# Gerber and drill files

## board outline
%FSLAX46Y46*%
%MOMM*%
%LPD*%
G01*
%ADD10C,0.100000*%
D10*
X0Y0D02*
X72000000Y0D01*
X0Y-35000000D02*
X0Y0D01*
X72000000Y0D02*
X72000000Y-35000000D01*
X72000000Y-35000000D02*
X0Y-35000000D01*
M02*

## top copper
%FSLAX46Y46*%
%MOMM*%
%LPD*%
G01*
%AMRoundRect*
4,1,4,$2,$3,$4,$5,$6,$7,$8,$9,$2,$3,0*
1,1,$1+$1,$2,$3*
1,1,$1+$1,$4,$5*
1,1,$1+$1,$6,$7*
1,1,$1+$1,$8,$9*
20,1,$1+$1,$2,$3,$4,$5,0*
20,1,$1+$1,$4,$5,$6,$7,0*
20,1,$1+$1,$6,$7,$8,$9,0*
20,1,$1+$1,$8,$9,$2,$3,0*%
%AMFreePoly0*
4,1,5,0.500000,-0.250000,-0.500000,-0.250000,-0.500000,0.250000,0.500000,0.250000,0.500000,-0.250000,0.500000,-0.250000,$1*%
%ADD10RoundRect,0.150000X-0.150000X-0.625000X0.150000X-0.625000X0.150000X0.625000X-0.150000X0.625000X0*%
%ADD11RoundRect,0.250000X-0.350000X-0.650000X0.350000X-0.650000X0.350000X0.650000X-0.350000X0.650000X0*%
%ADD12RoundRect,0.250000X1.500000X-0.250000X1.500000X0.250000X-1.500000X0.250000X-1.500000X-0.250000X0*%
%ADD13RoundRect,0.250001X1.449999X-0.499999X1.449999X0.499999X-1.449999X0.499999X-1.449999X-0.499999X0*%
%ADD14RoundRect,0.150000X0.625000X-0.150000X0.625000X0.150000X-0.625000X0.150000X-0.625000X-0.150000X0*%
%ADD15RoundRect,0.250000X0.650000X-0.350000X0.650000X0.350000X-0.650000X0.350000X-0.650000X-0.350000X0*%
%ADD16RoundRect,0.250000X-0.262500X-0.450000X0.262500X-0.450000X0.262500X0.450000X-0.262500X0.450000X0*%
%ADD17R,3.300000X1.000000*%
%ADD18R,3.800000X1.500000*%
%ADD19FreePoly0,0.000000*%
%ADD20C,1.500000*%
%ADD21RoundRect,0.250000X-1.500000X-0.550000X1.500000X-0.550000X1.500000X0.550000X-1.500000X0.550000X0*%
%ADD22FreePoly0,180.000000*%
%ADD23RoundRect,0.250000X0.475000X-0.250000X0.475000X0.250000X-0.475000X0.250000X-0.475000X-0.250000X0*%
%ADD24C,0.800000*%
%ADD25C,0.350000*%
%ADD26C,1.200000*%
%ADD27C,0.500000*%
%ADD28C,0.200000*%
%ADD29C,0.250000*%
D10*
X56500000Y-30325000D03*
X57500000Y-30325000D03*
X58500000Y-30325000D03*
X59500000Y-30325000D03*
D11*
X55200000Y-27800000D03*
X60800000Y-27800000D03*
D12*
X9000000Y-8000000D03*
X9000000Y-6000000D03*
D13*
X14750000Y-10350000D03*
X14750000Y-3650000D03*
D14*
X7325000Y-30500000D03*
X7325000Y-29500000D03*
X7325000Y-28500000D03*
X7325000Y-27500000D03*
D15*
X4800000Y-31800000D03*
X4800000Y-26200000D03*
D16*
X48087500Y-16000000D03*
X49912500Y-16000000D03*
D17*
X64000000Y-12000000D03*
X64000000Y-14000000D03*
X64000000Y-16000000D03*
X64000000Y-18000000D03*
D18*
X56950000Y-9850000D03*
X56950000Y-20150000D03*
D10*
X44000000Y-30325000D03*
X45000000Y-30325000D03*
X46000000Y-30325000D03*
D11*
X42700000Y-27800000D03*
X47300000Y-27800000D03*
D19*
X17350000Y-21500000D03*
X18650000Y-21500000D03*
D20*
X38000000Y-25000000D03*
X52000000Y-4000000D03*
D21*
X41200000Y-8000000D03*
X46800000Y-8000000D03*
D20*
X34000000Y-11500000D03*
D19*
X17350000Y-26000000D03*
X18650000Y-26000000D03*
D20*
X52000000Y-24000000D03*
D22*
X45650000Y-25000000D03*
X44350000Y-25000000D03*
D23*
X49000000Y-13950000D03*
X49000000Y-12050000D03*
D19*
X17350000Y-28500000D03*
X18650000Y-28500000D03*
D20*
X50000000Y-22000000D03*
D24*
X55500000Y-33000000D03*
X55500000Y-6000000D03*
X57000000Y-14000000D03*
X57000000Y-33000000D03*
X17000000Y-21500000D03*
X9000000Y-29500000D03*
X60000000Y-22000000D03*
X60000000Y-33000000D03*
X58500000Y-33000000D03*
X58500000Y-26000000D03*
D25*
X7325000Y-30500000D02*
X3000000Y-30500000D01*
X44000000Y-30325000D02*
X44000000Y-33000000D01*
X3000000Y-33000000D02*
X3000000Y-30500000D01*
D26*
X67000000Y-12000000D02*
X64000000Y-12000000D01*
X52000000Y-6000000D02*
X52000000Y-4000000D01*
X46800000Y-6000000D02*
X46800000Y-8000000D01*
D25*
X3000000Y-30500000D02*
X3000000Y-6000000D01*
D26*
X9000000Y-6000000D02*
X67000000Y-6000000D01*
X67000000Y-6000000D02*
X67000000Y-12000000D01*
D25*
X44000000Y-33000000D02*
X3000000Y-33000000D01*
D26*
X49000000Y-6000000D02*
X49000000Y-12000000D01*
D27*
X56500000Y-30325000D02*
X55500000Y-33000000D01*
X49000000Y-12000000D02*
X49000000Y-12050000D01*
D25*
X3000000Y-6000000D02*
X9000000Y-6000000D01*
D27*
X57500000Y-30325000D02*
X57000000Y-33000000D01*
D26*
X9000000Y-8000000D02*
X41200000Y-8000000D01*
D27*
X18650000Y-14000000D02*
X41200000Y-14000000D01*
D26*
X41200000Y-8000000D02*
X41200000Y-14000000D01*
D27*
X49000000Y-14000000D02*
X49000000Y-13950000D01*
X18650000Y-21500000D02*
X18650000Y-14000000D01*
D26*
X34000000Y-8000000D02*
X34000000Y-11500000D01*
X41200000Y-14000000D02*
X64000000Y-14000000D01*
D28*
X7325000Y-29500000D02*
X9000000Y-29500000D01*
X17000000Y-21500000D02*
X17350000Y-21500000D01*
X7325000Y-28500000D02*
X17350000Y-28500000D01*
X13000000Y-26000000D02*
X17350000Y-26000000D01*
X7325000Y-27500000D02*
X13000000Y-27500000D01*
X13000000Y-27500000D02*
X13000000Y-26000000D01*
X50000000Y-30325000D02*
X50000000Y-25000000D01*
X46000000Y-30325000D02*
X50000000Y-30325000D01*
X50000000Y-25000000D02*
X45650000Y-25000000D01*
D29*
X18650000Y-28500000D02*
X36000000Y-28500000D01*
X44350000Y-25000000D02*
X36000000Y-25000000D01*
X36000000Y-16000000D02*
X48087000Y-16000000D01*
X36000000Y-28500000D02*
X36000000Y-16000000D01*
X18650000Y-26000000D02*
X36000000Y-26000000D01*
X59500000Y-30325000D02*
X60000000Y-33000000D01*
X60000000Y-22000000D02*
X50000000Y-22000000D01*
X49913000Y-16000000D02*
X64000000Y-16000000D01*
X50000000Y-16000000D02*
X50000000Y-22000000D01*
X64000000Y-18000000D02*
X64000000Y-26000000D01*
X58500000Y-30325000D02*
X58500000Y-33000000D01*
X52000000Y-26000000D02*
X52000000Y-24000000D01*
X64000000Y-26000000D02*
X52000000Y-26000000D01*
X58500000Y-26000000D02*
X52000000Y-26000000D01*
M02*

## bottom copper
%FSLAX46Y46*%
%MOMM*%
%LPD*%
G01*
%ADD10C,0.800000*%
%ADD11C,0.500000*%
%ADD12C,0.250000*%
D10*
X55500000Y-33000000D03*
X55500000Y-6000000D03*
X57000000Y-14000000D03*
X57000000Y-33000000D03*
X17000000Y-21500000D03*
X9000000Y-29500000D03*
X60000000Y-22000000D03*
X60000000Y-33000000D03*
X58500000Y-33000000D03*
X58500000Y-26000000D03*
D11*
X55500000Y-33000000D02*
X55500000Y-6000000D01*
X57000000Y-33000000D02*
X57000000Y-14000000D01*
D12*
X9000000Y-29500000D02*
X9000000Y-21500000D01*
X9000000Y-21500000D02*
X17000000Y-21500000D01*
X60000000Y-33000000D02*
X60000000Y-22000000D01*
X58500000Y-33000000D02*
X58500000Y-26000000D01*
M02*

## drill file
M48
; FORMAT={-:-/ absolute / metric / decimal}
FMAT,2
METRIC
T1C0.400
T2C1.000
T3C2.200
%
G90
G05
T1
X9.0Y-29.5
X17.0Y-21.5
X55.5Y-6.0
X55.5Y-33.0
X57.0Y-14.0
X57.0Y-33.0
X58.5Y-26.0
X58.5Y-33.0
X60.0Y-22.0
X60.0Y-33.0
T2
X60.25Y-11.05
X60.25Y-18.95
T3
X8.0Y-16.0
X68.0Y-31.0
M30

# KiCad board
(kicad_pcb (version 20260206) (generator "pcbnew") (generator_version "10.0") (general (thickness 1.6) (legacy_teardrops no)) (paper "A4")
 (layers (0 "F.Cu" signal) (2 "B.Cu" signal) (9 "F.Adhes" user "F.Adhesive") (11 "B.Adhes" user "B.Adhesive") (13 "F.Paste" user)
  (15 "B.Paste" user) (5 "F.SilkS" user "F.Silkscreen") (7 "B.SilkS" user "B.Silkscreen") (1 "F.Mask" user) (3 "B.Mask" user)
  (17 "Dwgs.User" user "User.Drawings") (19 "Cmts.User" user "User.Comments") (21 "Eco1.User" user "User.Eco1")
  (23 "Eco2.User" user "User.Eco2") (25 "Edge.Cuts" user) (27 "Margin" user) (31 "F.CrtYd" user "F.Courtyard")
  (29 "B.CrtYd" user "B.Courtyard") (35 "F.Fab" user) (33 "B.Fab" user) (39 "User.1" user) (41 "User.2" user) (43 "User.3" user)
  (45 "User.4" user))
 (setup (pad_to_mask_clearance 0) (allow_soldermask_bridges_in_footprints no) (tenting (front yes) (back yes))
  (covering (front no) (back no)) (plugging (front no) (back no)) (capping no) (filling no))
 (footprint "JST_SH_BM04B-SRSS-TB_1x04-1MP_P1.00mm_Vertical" (layer "F.Cu") (at 58 29)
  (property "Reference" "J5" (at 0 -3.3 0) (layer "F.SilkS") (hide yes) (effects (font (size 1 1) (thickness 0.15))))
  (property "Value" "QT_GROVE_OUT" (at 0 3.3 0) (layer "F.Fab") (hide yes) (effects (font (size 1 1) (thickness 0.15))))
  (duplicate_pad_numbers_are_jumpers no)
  (pad "1" smd roundrect (at -1.5 1.325) (size 0.6 1.55) (layers "F.Cu" "F.Mask" "F.Paste") (roundrect_rratio 0.25) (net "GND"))
  (pad "2" smd roundrect (at -0.5 1.325) (size 0.6 1.55) (layers "F.Cu" "F.Mask" "F.Paste") (roundrect_rratio 0.25) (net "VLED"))
  (pad "3" smd roundrect (at 0.5 1.325) (size 0.6 1.55) (layers "F.Cu" "F.Mask" "F.Paste") (roundrect_rratio 0.25) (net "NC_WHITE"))
  (pad "4" smd roundrect (at 1.5 1.325) (size 0.6 1.55) (layers "F.Cu" "F.Mask" "F.Paste") (roundrect_rratio 0.25) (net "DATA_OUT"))
  (pad "MP" smd roundrect (at -2.8 -1.2) (size 1.2 1.8) (layers "F.Cu" "F.Mask" "F.Paste") (roundrect_rratio 0.208333))
  (pad "MP" smd roundrect (at 2.8 -1.2) (size 1.2 1.8) (layers "F.Cu" "F.Mask" "F.Paste") (roundrect_rratio 0.208333)))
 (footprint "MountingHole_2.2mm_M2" (layer "F.Cu") (at 68 31)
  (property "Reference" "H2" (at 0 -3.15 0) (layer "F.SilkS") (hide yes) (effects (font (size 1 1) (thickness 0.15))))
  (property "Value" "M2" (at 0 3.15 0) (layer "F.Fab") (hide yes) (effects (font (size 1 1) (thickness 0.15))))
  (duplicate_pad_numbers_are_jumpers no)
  (pad "" np_thru_hole circle (at 0 0) (size 2.2 2.2) (drill 2.2) (layers "*.Cu" "*.Mask")))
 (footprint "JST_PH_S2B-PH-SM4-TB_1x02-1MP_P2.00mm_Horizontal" (layer "F.Cu") (at 11.85 7 90)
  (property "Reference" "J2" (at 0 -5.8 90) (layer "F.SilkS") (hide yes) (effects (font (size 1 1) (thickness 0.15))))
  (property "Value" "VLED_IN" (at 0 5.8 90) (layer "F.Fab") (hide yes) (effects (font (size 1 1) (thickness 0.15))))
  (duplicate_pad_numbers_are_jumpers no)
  (pad "1" smd roundrect (at -1 -2.85 90) (size 1 3.5) (layers "F.Cu" "F.Mask" "F.Paste") (roundrect_rratio 0.25) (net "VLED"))
  (pad "2" smd roundrect (at 1 -2.85 90) (size 1 3.5) (layers "F.Cu" "F.Mask" "F.Paste") (roundrect_rratio 0.25) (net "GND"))
  (pad "MP" smd roundrect (at -3.35 2.9 90) (size 1.5 3.4) (layers "F.Cu" "F.Mask" "F.Paste") (roundrect_rratio 0.166667))
  (pad "MP" smd roundrect (at 3.35 2.9 90) (size 1.5 3.4) (layers "F.Cu" "F.Mask" "F.Paste") (roundrect_rratio 0.166667)))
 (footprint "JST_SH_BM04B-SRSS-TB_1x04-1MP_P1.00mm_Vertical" (layer "F.Cu") (at 6 29 90)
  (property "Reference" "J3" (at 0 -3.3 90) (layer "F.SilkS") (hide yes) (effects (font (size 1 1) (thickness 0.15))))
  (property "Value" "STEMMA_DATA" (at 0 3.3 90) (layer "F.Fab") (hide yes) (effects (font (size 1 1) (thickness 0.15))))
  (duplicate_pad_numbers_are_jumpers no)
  (pad "1" smd roundrect (at -1.5 1.325 90) (size 0.6 1.55) (layers "F.Cu" "F.Mask" "F.Paste") (roundrect_rratio 0.25) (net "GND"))
  (pad "2" smd roundrect (at -0.5 1.325 90) (size 0.6 1.55) (layers "F.Cu" "F.Mask" "F.Paste") (roundrect_rratio 0.25) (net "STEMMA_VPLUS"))
  (pad "3" smd roundrect (at 0.5 1.325 90) (size 0.6 1.55) (layers "F.Cu" "F.Mask" "F.Paste") (roundrect_rratio 0.25) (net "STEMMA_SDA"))
  (pad "4" smd roundrect (at 1.5 1.325 90) (size 0.6 1.55) (layers "F.Cu" "F.Mask" "F.Paste") (roundrect_rratio 0.25) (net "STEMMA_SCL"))
  (pad "MP" smd roundrect (at -2.8 -1.2 90) (size 1.2 1.8) (layers "F.Cu" "F.Mask" "F.Paste") (roundrect_rratio 0.208333))
  (pad "MP" smd roundrect (at 2.8 -1.2 90) (size 1.2 1.8) (layers "F.Cu" "F.Mask" "F.Paste") (roundrect_rratio 0.208333)))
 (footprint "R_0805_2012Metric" (layer "F.Cu") (at 49 16)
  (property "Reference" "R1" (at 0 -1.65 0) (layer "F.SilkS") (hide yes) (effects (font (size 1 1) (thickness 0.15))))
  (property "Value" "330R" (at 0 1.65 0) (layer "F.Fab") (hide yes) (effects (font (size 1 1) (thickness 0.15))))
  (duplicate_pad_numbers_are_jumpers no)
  (pad "1" smd roundrect (at -0.9125 0) (size 1.025 1.4) (layers "F.Cu" "F.Mask" "F.Paste") (roundrect_rratio 0.243902) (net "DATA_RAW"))
  (pad "2" smd roundrect (at 0.9125 0) (size 1.025 1.4) (layers "F.Cu" "F.Mask" "F.Paste") (roundrect_rratio 0.243902) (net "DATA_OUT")))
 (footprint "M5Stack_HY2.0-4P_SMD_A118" (layer "F.Cu") (at 64 12)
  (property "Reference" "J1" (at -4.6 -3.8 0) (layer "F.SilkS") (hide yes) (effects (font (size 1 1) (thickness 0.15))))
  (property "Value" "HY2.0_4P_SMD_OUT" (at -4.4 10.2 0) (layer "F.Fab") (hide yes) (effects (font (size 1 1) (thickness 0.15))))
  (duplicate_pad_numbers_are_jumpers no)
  (pad "" np_thru_hole circle (at -3.75 -0.95) (size 1 1) (drill 1) (layers "*.Cu" "*.Mask"))
  (pad "" np_thru_hole circle (at -3.75 6.95) (size 1 1) (drill 1) (layers "*.Cu" "*.Mask"))
  (pad "1" smd rect (at 0 0) (size 3.3 1) (layers "F.Cu" "F.Mask" "F.Paste") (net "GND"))
  (pad "2" smd rect (at 0 2) (size 3.3 1) (layers "F.Cu" "F.Mask" "F.Paste") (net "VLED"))
  (pad "3" smd rect (at 0 4) (size 3.3 1) (layers "F.Cu" "F.Mask" "F.Paste") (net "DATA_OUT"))
  (pad "4" smd rect (at 0 6) (size 3.3 1) (layers "F.Cu" "F.Mask" "F.Paste") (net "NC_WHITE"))
  (pad "MP" smd rect (at -7.05 -2.15) (size 3.8 1.5) (layers "F.Cu" "F.Mask" "F.Paste"))
  (pad "MP" smd rect (at -7.05 8.15) (size 3.8 1.5) (layers "F.Cu" "F.Mask" "F.Paste")))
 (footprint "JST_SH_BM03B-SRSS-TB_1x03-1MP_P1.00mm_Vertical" (layer "F.Cu") (at 45 29)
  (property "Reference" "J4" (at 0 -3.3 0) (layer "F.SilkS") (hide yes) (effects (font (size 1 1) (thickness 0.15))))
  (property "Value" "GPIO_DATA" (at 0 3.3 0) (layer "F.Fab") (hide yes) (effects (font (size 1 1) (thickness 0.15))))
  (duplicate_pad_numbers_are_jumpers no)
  (pad "1" smd roundrect (at -1 1.325) (size 0.6 1.55) (layers "F.Cu" "F.Mask" "F.Paste") (roundrect_rratio 0.25) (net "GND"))
  (pad "2" smd roundrect (at 0 1.325) (size 0.6 1.55) (layers "F.Cu" "F.Mask" "F.Paste") (roundrect_rratio 0.25) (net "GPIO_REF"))
  (pad "3" smd roundrect (at 1 1.325) (size 0.6 1.55) (layers "F.Cu" "F.Mask" "F.Paste") (roundrect_rratio 0.25) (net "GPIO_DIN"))
  (pad "MP" smd roundrect (at -2.3 -1.2) (size 1.2 1.8) (layers "F.Cu" "F.Mask" "F.Paste") (roundrect_rratio 0.208333))
  (pad "MP" smd roundrect (at 2.3 -1.2) (size 1.2 1.8) (layers "F.Cu" "F.Mask" "F.Paste") (roundrect_rratio 0.208333)))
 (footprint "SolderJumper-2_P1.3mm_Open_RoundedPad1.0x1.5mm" (layer "F.Cu") (at 18 21.5)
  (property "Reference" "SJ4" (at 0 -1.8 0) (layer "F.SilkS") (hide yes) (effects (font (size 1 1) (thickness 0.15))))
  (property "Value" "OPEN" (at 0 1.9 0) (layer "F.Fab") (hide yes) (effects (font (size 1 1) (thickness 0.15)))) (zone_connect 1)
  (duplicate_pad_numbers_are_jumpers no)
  (pad "1" smd custom (at -0.65 0) (size 1 0.5) (layers "F.Cu" "F.Mask") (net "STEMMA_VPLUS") (zone_connect 2) (thermal_bridge_angle 45)
   (options (clearance outline) (anchor rect)) (primitives))
  (pad "2" smd custom (at 0.65 0) (size 1 0.5) (layers "F.Cu" "F.Mask") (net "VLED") (zone_connect 2) (thermal_bridge_angle 45)
   (options (clearance outline) (anchor rect)) (primitives)))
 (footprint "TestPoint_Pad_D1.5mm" (layer "F.Cu") (at 38 25)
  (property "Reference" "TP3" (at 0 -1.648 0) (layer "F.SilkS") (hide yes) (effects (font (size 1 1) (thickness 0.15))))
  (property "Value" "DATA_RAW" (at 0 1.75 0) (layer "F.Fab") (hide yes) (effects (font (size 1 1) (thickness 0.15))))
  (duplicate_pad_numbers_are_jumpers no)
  (pad "1" smd circle (at 0 0) (size 1.5 1.5) (layers "F.Cu" "F.Mask") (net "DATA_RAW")))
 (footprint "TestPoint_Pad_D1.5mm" (layer "F.Cu") (at 52 4)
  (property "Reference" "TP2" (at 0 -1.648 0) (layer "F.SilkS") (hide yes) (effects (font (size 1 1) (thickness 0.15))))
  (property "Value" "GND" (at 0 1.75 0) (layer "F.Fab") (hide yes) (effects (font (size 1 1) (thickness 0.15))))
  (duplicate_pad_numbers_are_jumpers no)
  (pad "1" smd circle (at 0 0) (size 1.5 1.5) (layers "F.Cu" "F.Mask") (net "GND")))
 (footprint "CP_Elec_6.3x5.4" (layer "F.Cu") (at 44 8)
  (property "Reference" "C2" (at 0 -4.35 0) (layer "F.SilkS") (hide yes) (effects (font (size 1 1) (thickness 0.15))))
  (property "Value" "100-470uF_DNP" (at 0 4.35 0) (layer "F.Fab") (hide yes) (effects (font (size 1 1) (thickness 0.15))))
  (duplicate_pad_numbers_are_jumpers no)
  (pad "1" smd roundrect (at -2.8 0) (size 3.5 1.6) (layers "F.Cu" "F.Mask" "F.Paste") (roundrect_rratio 0.15625) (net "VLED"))
  (pad "2" smd roundrect (at 2.8 0) (size 3.5 1.6) (layers "F.Cu" "F.Mask" "F.Paste") (roundrect_rratio 0.15625) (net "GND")))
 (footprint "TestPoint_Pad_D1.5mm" (layer "F.Cu") (at 34 11.5)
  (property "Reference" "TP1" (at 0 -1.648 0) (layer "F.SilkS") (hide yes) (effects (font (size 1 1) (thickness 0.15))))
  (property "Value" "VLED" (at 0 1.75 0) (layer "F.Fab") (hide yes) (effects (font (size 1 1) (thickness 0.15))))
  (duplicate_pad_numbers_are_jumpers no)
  (pad "1" smd circle (at 0 0) (size 1.5 1.5) (layers "F.Cu" "F.Mask") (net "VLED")))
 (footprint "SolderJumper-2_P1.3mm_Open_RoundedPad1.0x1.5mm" (layer "F.Cu") (at 18 26)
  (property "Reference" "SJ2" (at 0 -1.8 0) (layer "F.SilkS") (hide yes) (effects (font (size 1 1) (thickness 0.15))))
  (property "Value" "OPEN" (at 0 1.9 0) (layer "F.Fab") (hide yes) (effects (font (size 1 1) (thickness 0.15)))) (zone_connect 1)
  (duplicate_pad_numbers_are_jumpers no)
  (pad "1" smd custom (at -0.65 0) (size 1 0.5) (layers "F.Cu" "F.Mask") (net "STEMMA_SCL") (zone_connect 2) (thermal_bridge_angle 45)
   (options (clearance outline) (anchor rect)) (primitives))
  (pad "2" smd custom (at 0.65 0) (size 1 0.5) (layers "F.Cu" "F.Mask") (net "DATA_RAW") (zone_connect 2) (thermal_bridge_angle 45)
   (options (clearance outline) (anchor rect)) (primitives)))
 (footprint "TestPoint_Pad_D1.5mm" (layer "F.Cu") (at 52 24)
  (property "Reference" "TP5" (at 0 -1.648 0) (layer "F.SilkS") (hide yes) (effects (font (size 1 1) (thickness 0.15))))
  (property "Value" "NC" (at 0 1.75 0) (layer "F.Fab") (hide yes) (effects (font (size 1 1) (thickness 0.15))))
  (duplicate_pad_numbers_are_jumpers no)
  (pad "1" smd circle (at 0 0) (size 1.5 1.5) (layers "F.Cu" "F.Mask") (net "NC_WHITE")))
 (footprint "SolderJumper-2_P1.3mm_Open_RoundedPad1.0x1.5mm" (layer "F.Cu") (at 45 25 180)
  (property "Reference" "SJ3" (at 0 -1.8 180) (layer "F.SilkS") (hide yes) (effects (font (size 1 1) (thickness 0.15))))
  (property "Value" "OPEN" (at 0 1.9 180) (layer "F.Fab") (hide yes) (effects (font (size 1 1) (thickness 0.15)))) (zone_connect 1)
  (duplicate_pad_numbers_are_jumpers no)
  (pad "1" smd custom (at -0.65 0 180) (size 1 0.5) (layers "F.Cu" "F.Mask") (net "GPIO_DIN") (zone_connect 2) (thermal_bridge_angle 45)
   (options (clearance outline) (anchor rect)) (primitives))
  (pad "2" smd custom (at 0.65 0 180) (size 1 0.5) (layers "F.Cu" "F.Mask") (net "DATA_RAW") (zone_connect 2) (thermal_bridge_angle 45)
   (options (clearance outline) (anchor rect)) (primitives)))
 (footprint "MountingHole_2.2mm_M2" (layer "F.Cu") (at 8 16)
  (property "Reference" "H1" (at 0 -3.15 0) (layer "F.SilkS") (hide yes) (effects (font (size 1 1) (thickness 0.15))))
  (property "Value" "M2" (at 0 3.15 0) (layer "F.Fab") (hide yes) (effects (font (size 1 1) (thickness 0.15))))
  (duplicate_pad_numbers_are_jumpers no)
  (pad "" np_thru_hole circle (at 0 0) (size 2.2 2.2) (drill 2.2) (layers "*.Cu" "*.Mask")))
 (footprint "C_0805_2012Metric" (layer "F.Cu") (at 49 13 90)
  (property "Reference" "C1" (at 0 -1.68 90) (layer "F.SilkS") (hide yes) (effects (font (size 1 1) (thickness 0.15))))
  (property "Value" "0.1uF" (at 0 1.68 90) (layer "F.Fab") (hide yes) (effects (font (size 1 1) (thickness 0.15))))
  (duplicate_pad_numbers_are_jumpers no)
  (pad "1" smd roundrect (at -0.95 0 90) (size 1 1.45) (layers "F.Cu" "F.Mask" "F.Paste") (roundrect_rratio 0.25) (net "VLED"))
  (pad "2" smd roundrect (at 0.95 0 90) (size 1 1.45) (layers "F.Cu" "F.Mask" "F.Paste") (roundrect_rratio 0.25) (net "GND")))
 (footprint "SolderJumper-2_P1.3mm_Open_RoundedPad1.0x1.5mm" (layer "F.Cu") (at 18 28.5)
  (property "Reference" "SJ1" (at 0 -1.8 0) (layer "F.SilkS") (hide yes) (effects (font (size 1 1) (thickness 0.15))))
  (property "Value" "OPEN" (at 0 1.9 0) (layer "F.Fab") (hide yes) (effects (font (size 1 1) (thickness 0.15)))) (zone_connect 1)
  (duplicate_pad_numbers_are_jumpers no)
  (pad "1" smd custom (at -0.65 0) (size 1 0.5) (layers "F.Cu" "F.Mask") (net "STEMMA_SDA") (zone_connect 2) (thermal_bridge_angle 45)
   (options (clearance outline) (anchor rect)) (primitives))
  (pad "2" smd custom (at 0.65 0) (size 1 0.5) (layers "F.Cu" "F.Mask") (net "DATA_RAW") (zone_connect 2) (thermal_bridge_angle 45)
   (options (clearance outline) (anchor rect)) (primitives)))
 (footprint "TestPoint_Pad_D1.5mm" (layer "F.Cu") (at 50 22)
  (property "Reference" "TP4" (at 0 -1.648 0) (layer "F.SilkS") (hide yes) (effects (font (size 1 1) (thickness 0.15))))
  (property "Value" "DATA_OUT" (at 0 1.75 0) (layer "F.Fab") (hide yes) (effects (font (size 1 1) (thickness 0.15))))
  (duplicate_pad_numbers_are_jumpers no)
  (pad "1" smd circle (at 0 0) (size 1.5 1.5) (layers "F.Cu" "F.Mask") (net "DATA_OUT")))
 (gr_line (start 0 0) (end 72 0) (stroke (width 0.1) (type default)) (layer "Edge.Cuts"))
 (gr_line (start 0 35) (end 0 0) (stroke (width 0.1) (type default)) (layer "Edge.Cuts"))
 (gr_line (start 72 0) (end 72 35) (stroke (width 0.1) (type default)) (layer "Edge.Cuts"))
 (gr_line (start 72 35) (end 0 35) (stroke (width 0.1) (type default)) (layer "Edge.Cuts"))
 (segment (start 7.325 30.5) (end 3 30.5) (width 0.35) (layer "F.Cu") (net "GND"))
 (segment (start 44 30.325) (end 44 33) (width 0.35) (layer "F.Cu") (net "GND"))
 (segment (start 3 33) (end 3 30.5) (width 0.35) (layer "F.Cu") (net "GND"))
 (segment (start 67 12) (end 64 12) (width 1.2) (layer "F.Cu") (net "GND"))
 (segment (start 52 6) (end 52 4) (width 1.2) (layer "F.Cu") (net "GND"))
 (segment (start 46.8 6) (end 46.8 8) (width 1.2) (layer "F.Cu") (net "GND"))
 (segment (start 3 30.5) (end 3 6) (width 0.35) (layer "F.Cu") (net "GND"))
 (segment (start 9 6) (end 67 6) (width 1.2) (layer "F.Cu") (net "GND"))
 (segment (start 67 6) (end 67 12) (width 1.2) (layer "F.Cu") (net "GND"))
 (segment (start 44 33) (end 3 33) (width 0.35) (layer "F.Cu") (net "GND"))
 (segment (start 49 6) (end 49 12) (width 1.2) (layer "F.Cu") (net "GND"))
 (segment (start 56.5 30.325) (end 55.5 33) (width 0.5) (layer "F.Cu") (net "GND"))
 (segment (start 49 12) (end 49 12.05) (width 0.5) (layer "F.Cu") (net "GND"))
 (segment (start 3 6) (end 9 6) (width 0.35) (layer "F.Cu") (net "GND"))
 (via (at 55.5 33) (size 0.8) (drill 0.4) (layers "F.Cu" "B.Cu") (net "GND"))
 (via (at 55.5 6) (size 0.8) (drill 0.4) (layers "F.Cu" "B.Cu") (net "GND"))
 (segment (start 55.5 33) (end 55.5 6) (width 0.5) (layer "B.Cu") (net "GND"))
 (segment (start 57.5 30.325) (end 57 33) (width 0.5) (layer "F.Cu") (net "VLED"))
 (segment (start 9 8) (end 41.2 8) (width 1.2) (layer "F.Cu") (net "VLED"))
 (segment (start 18.65 14) (end 41.2 14) (width 0.5) (layer "F.Cu") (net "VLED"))
 (segment (start 41.2 8) (end 41.2 14) (width 1.2) (layer "F.Cu") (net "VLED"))
 (segment (start 49 14) (end 49 13.95) (width 0.5) (layer "F.Cu") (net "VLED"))
 (segment (start 18.65 21.5) (end 18.65 14) (width 0.5) (layer "F.Cu") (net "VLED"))
 (segment (start 34 8) (end 34 11.5) (width 1.2) (layer "F.Cu") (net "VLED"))
 (segment (start 41.2 14) (end 64 14) (width 1.2) (layer "F.Cu") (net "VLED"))
 (via (at 57 14) (size 0.8) (drill 0.4) (layers "F.Cu" "B.Cu") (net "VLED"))
 (via (at 57 33) (size 0.8) (drill 0.4) (layers "F.Cu" "B.Cu") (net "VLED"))
 (segment (start 57 33) (end 57 14) (width 0.5) (layer "B.Cu") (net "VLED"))
 (segment (start 7.325 29.5) (end 9 29.5) (width 0.2) (layer "F.Cu") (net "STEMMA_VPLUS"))
 (segment (start 17 21.5) (end 17.35 21.5) (width 0.2) (layer "F.Cu") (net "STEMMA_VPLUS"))
 (via (at 17 21.5) (size 0.8) (drill 0.4) (layers "F.Cu" "B.Cu") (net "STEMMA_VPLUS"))
 (via (at 9 29.5) (size 0.8) (drill 0.4) (layers "F.Cu" "B.Cu") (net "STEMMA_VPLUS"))
 (segment (start 9 29.5) (end 9 21.5) (width 0.25) (layer "B.Cu") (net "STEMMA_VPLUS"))
 (segment (start 9 21.5) (end 17 21.5) (width 0.25) (layer "B.Cu") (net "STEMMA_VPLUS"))
 (segment (start 7.325 28.5) (end 17.35 28.5) (width 0.2) (layer "F.Cu") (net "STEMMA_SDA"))
 (segment (start 13 26) (end 17.35 26) (width 0.2) (layer "F.Cu") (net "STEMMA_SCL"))
 (segment (start 7.325 27.5) (end 13 27.5) (width 0.2) (layer "F.Cu") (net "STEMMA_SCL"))
 (segment (start 13 27.5) (end 13 26) (width 0.2) (layer "F.Cu") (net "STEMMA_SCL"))
 (segment (start 50 30.325) (end 50 25) (width 0.2) (layer "F.Cu") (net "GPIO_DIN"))
 (segment (start 46 30.325) (end 50 30.325) (width 0.2) (layer "F.Cu") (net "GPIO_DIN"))
 (segment (start 50 25) (end 45.65 25) (width 0.2) (layer "F.Cu") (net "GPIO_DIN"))
 (segment (start 18.65 28.5) (end 36 28.5) (width 0.25) (layer "F.Cu") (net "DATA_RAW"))
 (segment (start 44.35 25) (end 36 25) (width 0.25) (layer "F.Cu") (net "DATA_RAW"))
 (segment (start 36 16) (end 48.087 16) (width 0.25) (layer "F.Cu") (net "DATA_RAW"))
 (segment (start 36 28.5) (end 36 16) (width 0.25) (layer "F.Cu") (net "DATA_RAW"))
 (segment (start 18.65 26) (end 36 26) (width 0.25) (layer "F.Cu") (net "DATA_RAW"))
 (segment (start 59.5 30.325) (end 60 33) (width 0.25) (layer "F.Cu") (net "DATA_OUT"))
 (segment (start 60 22) (end 50 22) (width 0.25) (layer "F.Cu") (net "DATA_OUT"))
 (segment (start 49.913 16) (end 64 16) (width 0.25) (layer "F.Cu") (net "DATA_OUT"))
 (segment (start 50 16) (end 50 22) (width 0.25) (layer "F.Cu") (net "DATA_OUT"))
 (via (at 60 22) (size 0.8) (drill 0.4) (layers "F.Cu" "B.Cu") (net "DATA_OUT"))
 (via (at 60 33) (size 0.8) (drill 0.4) (layers "F.Cu" "B.Cu") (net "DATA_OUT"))
 (segment (start 60 33) (end 60 22) (width 0.25) (layer "B.Cu") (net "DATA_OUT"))
 (segment (start 64 18) (end 64 26) (width 0.25) (layer "F.Cu") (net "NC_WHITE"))
 (segment (start 58.5 30.325) (end 58.5 33) (width 0.25) (layer "F.Cu") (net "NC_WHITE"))
 (segment (start 52 26) (end 52 24) (width 0.25) (layer "F.Cu") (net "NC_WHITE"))
 (segment (start 64 26) (end 52 26) (width 0.25) (layer "F.Cu") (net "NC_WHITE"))
 (segment (start 58.5 26) (end 52 26) (width 0.25) (layer "F.Cu") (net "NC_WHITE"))
 (via (at 58.5 33) (size 0.8) (drill 0.4) (layers "F.Cu" "B.Cu") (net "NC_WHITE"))
 (via (at 58.5 26) (size 0.8) (drill 0.4) (layers "F.Cu" "B.Cu") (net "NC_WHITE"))
 (segment (start 58.5 33) (end 58.5 26) (width 0.25) (layer "B.Cu") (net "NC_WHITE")))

